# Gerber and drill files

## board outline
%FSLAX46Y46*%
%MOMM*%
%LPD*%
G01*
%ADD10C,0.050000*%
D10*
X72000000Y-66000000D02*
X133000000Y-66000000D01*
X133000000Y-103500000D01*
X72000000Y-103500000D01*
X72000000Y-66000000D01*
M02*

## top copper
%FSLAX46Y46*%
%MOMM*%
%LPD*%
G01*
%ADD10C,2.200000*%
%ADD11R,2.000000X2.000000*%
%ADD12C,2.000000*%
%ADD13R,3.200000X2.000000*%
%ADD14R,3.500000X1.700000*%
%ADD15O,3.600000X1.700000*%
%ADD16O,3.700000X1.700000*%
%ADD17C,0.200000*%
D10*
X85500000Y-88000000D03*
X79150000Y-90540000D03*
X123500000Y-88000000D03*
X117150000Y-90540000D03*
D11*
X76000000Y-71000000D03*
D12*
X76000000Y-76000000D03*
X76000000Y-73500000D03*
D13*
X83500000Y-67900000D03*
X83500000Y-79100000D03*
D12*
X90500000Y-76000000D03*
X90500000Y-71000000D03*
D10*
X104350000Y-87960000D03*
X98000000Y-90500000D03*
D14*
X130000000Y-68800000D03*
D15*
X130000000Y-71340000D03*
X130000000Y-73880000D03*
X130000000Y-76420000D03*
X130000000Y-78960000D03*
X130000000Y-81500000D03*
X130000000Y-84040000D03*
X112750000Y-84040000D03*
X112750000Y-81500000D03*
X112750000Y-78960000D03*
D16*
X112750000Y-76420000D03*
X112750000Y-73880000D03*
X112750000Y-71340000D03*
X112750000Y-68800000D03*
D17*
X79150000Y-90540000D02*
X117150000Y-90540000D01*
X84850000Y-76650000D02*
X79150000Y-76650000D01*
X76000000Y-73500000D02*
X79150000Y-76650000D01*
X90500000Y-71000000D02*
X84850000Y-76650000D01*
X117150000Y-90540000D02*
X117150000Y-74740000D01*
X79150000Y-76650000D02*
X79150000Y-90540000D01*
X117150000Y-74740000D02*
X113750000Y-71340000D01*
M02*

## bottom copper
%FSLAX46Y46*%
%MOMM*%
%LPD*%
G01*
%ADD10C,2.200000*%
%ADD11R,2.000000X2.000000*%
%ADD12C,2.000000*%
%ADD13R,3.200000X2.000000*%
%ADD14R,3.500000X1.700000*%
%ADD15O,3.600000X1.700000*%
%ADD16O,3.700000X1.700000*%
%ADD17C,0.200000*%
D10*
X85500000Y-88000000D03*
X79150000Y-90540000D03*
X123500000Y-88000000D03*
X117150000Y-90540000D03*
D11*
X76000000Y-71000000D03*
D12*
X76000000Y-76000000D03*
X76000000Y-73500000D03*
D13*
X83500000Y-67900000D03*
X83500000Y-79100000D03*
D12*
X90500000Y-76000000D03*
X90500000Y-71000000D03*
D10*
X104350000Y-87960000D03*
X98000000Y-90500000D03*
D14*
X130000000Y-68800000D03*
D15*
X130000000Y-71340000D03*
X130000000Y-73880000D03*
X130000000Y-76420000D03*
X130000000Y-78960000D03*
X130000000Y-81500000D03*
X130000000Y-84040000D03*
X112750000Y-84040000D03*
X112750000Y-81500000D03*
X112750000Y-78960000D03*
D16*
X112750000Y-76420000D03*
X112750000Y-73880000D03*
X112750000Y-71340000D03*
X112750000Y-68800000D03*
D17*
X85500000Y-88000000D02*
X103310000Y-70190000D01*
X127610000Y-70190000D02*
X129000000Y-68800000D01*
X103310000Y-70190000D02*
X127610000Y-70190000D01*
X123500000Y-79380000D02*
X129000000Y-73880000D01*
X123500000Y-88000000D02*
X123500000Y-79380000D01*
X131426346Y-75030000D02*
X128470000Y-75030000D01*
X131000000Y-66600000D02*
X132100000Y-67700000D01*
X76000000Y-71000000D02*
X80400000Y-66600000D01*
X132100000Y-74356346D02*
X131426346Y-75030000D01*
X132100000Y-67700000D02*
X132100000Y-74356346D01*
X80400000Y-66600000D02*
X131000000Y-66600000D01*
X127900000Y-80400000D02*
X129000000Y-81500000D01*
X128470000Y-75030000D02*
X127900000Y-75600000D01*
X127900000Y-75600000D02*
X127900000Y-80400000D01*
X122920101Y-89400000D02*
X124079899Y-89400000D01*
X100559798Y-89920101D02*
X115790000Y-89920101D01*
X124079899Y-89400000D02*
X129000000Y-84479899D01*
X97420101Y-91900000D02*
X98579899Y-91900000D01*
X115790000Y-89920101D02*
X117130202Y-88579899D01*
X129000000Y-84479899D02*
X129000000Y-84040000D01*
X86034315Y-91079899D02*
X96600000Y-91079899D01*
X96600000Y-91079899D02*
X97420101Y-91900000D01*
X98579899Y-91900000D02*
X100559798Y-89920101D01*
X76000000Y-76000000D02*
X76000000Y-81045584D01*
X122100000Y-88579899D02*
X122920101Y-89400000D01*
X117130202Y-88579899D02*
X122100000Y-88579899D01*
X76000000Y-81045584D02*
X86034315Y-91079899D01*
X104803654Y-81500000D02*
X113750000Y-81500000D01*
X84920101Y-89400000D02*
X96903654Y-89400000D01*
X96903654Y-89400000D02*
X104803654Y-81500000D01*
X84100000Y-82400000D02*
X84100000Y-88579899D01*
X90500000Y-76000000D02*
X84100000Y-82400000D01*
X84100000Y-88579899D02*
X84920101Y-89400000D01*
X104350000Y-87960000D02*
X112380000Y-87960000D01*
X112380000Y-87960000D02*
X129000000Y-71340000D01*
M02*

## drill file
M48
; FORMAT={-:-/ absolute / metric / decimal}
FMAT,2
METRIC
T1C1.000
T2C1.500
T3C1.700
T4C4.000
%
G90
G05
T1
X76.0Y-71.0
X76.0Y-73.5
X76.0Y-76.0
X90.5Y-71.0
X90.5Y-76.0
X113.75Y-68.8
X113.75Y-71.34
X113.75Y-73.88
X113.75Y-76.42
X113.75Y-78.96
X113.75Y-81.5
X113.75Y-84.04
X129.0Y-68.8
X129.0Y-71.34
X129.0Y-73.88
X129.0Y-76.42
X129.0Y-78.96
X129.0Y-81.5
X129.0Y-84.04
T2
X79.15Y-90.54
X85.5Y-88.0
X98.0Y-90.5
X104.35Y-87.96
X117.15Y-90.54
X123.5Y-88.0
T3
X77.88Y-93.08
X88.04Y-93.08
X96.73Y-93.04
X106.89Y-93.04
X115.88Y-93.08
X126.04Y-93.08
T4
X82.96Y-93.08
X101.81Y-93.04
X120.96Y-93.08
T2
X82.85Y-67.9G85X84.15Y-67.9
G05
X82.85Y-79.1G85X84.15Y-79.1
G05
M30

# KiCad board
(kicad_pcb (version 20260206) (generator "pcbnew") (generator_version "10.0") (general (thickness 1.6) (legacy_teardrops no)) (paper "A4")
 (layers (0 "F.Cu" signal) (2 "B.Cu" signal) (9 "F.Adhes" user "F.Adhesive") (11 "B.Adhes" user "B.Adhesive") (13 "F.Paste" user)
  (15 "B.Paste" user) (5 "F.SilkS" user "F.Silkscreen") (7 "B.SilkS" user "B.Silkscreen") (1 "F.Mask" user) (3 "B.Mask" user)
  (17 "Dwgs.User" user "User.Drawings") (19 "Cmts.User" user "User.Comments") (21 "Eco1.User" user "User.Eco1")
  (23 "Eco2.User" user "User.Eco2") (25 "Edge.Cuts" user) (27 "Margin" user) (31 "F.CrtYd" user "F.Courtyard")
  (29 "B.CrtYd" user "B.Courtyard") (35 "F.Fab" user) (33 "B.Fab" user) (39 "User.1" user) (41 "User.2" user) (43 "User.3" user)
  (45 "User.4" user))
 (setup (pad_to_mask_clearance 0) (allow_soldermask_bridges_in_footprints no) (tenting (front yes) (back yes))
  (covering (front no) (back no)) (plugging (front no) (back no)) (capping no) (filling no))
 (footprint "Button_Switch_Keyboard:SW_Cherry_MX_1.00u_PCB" (layer "F.Cu") (at 85.5 88)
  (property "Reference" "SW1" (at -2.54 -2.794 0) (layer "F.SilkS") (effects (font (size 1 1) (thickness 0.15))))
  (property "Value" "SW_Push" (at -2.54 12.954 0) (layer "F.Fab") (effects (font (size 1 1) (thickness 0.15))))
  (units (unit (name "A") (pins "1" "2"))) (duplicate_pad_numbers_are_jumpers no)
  (pad "" np_thru_hole circle (at -7.62 5.08) (size 1.7 1.7) (drill 1.7) (layers "*.Cu" "*.Mask"))
  (pad "" np_thru_hole circle (at -2.54 5.08) (size 4 4) (drill 4) (layers "*.Cu" "*.Mask"))
  (pad "" np_thru_hole circle (at 2.54 5.08) (size 1.7 1.7) (drill 1.7) (layers "*.Cu" "*.Mask"))
  (pad "1" thru_hole circle (at 0 0) (size 2.2 2.2) (drill 1.5) (layers "*.Cu" "*.Mask") (remove_unused_layers no)
   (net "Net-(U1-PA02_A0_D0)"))
  (pad "2" thru_hole circle (at -6.35 2.54) (size 2.2 2.2) (drill 1.5) (layers "*.Cu" "*.Mask") (remove_unused_layers no) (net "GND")))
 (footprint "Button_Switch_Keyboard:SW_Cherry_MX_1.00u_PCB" (layer "F.Cu") (at 123.5 88)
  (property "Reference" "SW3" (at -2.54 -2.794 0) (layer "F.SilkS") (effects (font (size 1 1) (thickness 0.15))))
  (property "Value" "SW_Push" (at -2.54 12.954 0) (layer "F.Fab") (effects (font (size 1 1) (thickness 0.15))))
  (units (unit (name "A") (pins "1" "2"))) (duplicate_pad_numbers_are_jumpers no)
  (pad "" np_thru_hole circle (at -7.62 5.08) (size 1.7 1.7) (drill 1.7) (layers "*.Cu" "*.Mask"))
  (pad "" np_thru_hole circle (at -2.54 5.08) (size 4 4) (drill 4) (layers "*.Cu" "*.Mask"))
  (pad "" np_thru_hole circle (at 2.54 5.08) (size 1.7 1.7) (drill 1.7) (layers "*.Cu" "*.Mask"))
  (pad "1" thru_hole circle (at 0 0) (size 2.2 2.2) (drill 1.5) (layers "*.Cu" "*.Mask") (remove_unused_layers no)
   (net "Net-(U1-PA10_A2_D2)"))
  (pad "2" thru_hole circle (at -6.35 2.54) (size 2.2 2.2) (drill 1.5) (layers "*.Cu" "*.Mask") (remove_unused_layers no) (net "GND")))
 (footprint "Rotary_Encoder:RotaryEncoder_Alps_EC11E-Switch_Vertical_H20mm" (layer "F.Cu") (at 76 71)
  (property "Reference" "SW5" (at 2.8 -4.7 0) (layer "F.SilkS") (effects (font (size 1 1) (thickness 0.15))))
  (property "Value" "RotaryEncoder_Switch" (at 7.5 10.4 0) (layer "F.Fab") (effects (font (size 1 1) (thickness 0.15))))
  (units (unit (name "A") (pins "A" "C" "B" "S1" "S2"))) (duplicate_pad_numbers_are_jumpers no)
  (pad "A" thru_hole rect (at 0 0) (size 2 2) (drill 1) (layers "*.Cu" "*.Mask") (remove_unused_layers no) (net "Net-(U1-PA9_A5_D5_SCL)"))
  (pad "B" thru_hole circle (at 0 5) (size 2 2) (drill 1) (layers "*.Cu" "*.Mask") (remove_unused_layers no) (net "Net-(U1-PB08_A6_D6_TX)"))
  (pad "C" thru_hole circle (at 0 2.5) (size 2 2) (drill 1) (layers "*.Cu" "*.Mask") (remove_unused_layers no) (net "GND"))
  (pad "MP" thru_hole rect (at 7.5 -3.1) (size 3.2 2) (drill oval 2.8 1.5) (layers "*.Cu" "*.Mask") (remove_unused_layers no))
  (pad "MP" thru_hole rect (at 7.5 8.1) (size 3.2 2) (drill oval 2.8 1.5) (layers "*.Cu" "*.Mask") (remove_unused_layers no))
  (pad "S1" thru_hole circle (at 14.5 5) (size 2 2) (drill 1) (layers "*.Cu" "*.Mask") (remove_unused_layers no)
   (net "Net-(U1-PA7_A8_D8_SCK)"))
  (pad "S2" thru_hole circle (at 14.5 0) (size 2 2) (drill 1) (layers "*.Cu" "*.Mask") (remove_unused_layers no) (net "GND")))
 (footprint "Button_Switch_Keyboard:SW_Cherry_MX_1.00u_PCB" (layer "F.Cu") (at 104.35 87.96)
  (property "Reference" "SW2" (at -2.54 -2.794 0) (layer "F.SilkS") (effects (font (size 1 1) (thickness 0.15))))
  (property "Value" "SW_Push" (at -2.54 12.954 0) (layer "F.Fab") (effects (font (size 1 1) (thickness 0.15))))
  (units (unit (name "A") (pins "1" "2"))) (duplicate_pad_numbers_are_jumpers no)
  (pad "" np_thru_hole circle (at -7.62 5.08) (size 1.7 1.7) (drill 1.7) (layers "*.Cu" "*.Mask"))
  (pad "" np_thru_hole circle (at -2.54 5.08) (size 4 4) (drill 4) (layers "*.Cu" "*.Mask"))
  (pad "" np_thru_hole circle (at 2.54 5.08) (size 1.7 1.7) (drill 1.7) (layers "*.Cu" "*.Mask"))
  (pad "1" thru_hole circle (at 0 0) (size 2.2 2.2) (drill 1.5) (layers "*.Cu" "*.Mask") (remove_unused_layers no)
   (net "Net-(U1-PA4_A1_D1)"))
  (pad "2" thru_hole circle (at -6.35 2.54) (size 2.2 2.2) (drill 1.5) (layers "*.Cu" "*.Mask") (remove_unused_layers no) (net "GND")))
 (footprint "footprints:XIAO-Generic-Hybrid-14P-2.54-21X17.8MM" (layer "B.Cu") (at 121.375 76.42 180)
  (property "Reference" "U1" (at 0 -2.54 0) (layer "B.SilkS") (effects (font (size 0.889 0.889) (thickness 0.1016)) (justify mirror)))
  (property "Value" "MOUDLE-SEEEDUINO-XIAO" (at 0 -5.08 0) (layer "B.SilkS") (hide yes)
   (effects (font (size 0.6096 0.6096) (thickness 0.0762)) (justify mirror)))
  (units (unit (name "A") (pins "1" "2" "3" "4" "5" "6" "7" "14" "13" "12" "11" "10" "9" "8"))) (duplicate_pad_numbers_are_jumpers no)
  (pad "1" thru_hole rect (at -7.625 7.62 180) (size 3.5 1.7) (drill 1 (offset -1 0)) (layers "*.Cu" "*.Mask") (remove_unused_layers no)
   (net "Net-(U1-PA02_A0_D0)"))
  (pad "2" thru_hole oval (at -7.625 5.08 180) (size 3.6 1.7) (drill 1 (offset -1 0)) (layers "*.Cu" "*.Mask") (remove_unused_layers no)
   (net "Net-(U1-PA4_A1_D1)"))
  (pad "3" thru_hole oval (at -7.625 2.54 180) (size 3.6 1.7) (drill 1 (offset -1 0)) (layers "*.Cu" "*.Mask") (remove_unused_layers no)
   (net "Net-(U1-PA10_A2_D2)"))
  (pad "4" thru_hole oval (at -7.625 0 180) (size 3.6 1.7) (drill 1 (offset -1 0)) (layers "*.Cu" "*.Mask") (remove_unused_layers no)
   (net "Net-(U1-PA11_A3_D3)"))
  (pad "5" thru_hole oval (at -7.625 -2.54 180) (size 3.6 1.7) (drill 1 (offset -1 0)) (layers "*.Cu" "*.Mask") (remove_unused_layers no)
   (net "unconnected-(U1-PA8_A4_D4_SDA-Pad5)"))
  (pad "6" thru_hole oval (at -7.625 -5.08) (size 3.6 1.7) (drill 1 (offset 1 0)) (layers "*.Cu" "*.Mask") (remove_unused_layers no)
   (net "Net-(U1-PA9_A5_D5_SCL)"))
  (pad "7" thru_hole oval (at -7.625 -7.62 180) (size 3.6 1.7) (drill 1 (offset -1 0)) (layers "*.Cu" "*.Mask") (remove_unused_layers no)
   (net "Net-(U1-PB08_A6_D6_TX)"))
  (pad "8" thru_hole oval (at 7.625 -7.62 180) (size 3.6 1.7) (drill 1 (offset 1 0)) (layers "*.Cu" "*.Mask") (remove_unused_layers no)
   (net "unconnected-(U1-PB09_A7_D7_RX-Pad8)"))
  (pad "9" thru_hole oval (at 7.625 -5.08 180) (size 3.6 1.7) (drill 1 (offset 1 0)) (layers "*.Cu" "*.Mask") (remove_unused_layers no)
   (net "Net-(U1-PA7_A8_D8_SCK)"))
  (pad "10" thru_hole oval (at 7.625 -2.54 180) (size 3.6 1.7) (drill 1 (offset 1 0)) (layers "*.Cu" "*.Mask") (remove_unused_layers no)
   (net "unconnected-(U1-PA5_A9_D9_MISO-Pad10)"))
  (pad "11" thru_hole oval (at 7.625 0 180) (size 3.7 1.7) (drill 1 (offset 1 0)) (layers "*.Cu" "*.Mask") (remove_unused_layers no)
   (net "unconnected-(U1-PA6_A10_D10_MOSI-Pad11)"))
  (pad "12" thru_hole oval (at 7.625 2.54 180) (size 3.7 1.7) (drill 1 (offset 1 0)) (layers "*.Cu" "*.Mask") (remove_unused_layers no)
   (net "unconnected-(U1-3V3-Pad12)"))
  (pad "13" thru_hole oval (at 7.625 5.08 180) (size 3.7 1.7) (drill 1 (offset 1 0)) (layers "*.Cu" "*.Mask") (remove_unused_layers no)
   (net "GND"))
  (pad "14" thru_hole oval (at 7.625 7.62 180) (size 3.7 1.7) (drill 1 (offset 1 0)) (layers "*.Cu" "*.Mask") (remove_unused_layers no)
   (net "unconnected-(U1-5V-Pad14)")))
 (gr_rect (start 72 66) (end 133 103.5) (stroke (width 0.05) (type default)) (fill no) (layer "Edge.Cuts"))
 (segment (start 85.5 88) (end 103.31 70.19) (width 0.2) (layer "B.Cu") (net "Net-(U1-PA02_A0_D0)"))
 (segment (start 127.61 70.19) (end 129 68.8) (width 0.2) (layer "B.Cu") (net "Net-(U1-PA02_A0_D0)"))
 (segment (start 103.31 70.19) (end 127.61 70.19) (width 0.2) (layer "B.Cu") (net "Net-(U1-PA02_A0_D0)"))
 (segment (start 79.15 90.54) (end 117.15 90.54) (width 0.2) (layer "F.Cu") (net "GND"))
 (segment (start 84.85 76.65) (end 79.15 76.65) (width 0.2) (layer "F.Cu") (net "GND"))
 (segment (start 76 73.5) (end 79.15 76.65) (width 0.2) (layer "F.Cu") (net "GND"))
 (segment (start 90.5 71) (end 84.85 76.65) (width 0.2) (layer "F.Cu") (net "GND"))
 (segment (start 117.15 90.54) (end 117.15 74.74) (width 0.2) (layer "F.Cu") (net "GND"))
 (segment (start 79.15 76.65) (end 79.15 90.54) (width 0.2) (layer "F.Cu") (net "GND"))
 (segment (start 117.15 74.74) (end 113.75 71.34) (width 0.2) (layer "F.Cu") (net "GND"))
 (segment (start 123.5 79.38) (end 129 73.88) (width 0.2) (layer "B.Cu") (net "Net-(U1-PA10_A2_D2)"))
 (segment (start 123.5 88) (end 123.5 79.38) (width 0.2) (layer "B.Cu") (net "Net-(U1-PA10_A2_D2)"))
 (segment (start 131.426346 75.03) (end 128.47 75.03) (width 0.2) (layer "B.Cu") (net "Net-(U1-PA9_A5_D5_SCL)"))
 (segment (start 131 66.6) (end 132.1 67.7) (width 0.2) (layer "B.Cu") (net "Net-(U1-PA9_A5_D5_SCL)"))
 (segment (start 76 71) (end 80.4 66.6) (width 0.2) (layer "B.Cu") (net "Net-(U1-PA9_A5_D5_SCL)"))
 (segment (start 132.1 74.356346) (end 131.426346 75.03) (width 0.2) (layer "B.Cu") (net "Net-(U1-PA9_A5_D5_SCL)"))
 (segment (start 132.1 67.7) (end 132.1 74.356346) (width 0.2) (layer "B.Cu") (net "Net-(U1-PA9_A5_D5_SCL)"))
 (segment (start 80.4 66.6) (end 131 66.6) (width 0.2) (layer "B.Cu") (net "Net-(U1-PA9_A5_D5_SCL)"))
 (segment (start 127.9 80.4) (end 129 81.5) (width 0.2) (layer "B.Cu") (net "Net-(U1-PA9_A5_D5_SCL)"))
 (segment (start 128.47 75.03) (end 127.9 75.6) (width 0.2) (layer "B.Cu") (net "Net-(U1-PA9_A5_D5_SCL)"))
 (segment (start 127.9 75.6) (end 127.9 80.4) (width 0.2) (layer "B.Cu") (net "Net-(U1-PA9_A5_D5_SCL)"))
 (segment (start 122.920101 89.4) (end 124.079899 89.4) (width 0.2) (layer "B.Cu") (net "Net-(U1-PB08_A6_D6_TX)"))
 (segment (start 100.559798 89.920101) (end 115.79 89.920101) (width 0.2) (layer "B.Cu") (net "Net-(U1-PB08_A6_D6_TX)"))
 (segment (start 124.079899 89.4) (end 129 84.479899) (width 0.2) (layer "B.Cu") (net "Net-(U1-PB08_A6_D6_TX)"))
 (segment (start 97.420101 91.9) (end 98.579899 91.9) (width 0.2) (layer "B.Cu") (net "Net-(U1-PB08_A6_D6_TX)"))
 (segment (start 115.79 89.920101) (end 117.130202 88.579899) (width 0.2) (layer "B.Cu") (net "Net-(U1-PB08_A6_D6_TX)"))
 (segment (start 129 84.479899) (end 129 84.04) (width 0.2) (layer "B.Cu") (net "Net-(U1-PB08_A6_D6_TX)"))
 (segment (start 86.034315 91.079899) (end 96.6 91.079899) (width 0.2) (layer "B.Cu") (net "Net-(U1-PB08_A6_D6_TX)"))
 (segment (start 96.6 91.079899) (end 97.420101 91.9) (width 0.2) (layer "B.Cu") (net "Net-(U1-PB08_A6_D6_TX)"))
 (segment (start 98.579899 91.9) (end 100.559798 89.920101) (width 0.2) (layer "B.Cu") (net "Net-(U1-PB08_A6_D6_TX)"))
 (segment (start 76 76) (end 76 81.045584) (width 0.2) (layer "B.Cu") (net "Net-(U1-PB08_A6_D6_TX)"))
 (segment (start 122.1 88.579899) (end 122.920101 89.4) (width 0.2) (layer "B.Cu") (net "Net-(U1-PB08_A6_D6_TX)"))
 (segment (start 117.130202 88.579899) (end 122.1 88.579899) (width 0.2) (layer "B.Cu") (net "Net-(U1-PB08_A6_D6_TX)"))
 (segment (start 76 81.045584) (end 86.034315 91.079899) (width 0.2) (layer "B.Cu") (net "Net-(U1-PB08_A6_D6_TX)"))
 (segment (start 104.803654 81.5) (end 113.75 81.5) (width 0.2) (layer "B.Cu") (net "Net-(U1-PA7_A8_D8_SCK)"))
 (segment (start 84.920101 89.4) (end 96.903654 89.4) (width 0.2) (layer "B.Cu") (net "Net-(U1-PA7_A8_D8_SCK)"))
 (segment (start 96.903654 89.4) (end 104.803654 81.5) (width 0.2) (layer "B.Cu") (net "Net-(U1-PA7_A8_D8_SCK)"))
 (segment (start 84.1 82.4) (end 84.1 88.579899) (width 0.2) (layer "B.Cu") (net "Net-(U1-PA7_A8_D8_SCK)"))
 (segment (start 90.5 76) (end 84.1 82.4) (width 0.2) (layer "B.Cu") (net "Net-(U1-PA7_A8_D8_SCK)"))
 (segment (start 84.1 88.579899) (end 84.920101 89.4) (width 0.2) (layer "B.Cu") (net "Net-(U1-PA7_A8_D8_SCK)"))
 (segment (start 104.35 87.96) (end 112.38 87.96) (width 0.2) (layer "B.Cu") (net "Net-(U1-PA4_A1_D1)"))
 (segment (start 112.38 87.96) (end 129 71.34) (width 0.2) (layer "B.Cu") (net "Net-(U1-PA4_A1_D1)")))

